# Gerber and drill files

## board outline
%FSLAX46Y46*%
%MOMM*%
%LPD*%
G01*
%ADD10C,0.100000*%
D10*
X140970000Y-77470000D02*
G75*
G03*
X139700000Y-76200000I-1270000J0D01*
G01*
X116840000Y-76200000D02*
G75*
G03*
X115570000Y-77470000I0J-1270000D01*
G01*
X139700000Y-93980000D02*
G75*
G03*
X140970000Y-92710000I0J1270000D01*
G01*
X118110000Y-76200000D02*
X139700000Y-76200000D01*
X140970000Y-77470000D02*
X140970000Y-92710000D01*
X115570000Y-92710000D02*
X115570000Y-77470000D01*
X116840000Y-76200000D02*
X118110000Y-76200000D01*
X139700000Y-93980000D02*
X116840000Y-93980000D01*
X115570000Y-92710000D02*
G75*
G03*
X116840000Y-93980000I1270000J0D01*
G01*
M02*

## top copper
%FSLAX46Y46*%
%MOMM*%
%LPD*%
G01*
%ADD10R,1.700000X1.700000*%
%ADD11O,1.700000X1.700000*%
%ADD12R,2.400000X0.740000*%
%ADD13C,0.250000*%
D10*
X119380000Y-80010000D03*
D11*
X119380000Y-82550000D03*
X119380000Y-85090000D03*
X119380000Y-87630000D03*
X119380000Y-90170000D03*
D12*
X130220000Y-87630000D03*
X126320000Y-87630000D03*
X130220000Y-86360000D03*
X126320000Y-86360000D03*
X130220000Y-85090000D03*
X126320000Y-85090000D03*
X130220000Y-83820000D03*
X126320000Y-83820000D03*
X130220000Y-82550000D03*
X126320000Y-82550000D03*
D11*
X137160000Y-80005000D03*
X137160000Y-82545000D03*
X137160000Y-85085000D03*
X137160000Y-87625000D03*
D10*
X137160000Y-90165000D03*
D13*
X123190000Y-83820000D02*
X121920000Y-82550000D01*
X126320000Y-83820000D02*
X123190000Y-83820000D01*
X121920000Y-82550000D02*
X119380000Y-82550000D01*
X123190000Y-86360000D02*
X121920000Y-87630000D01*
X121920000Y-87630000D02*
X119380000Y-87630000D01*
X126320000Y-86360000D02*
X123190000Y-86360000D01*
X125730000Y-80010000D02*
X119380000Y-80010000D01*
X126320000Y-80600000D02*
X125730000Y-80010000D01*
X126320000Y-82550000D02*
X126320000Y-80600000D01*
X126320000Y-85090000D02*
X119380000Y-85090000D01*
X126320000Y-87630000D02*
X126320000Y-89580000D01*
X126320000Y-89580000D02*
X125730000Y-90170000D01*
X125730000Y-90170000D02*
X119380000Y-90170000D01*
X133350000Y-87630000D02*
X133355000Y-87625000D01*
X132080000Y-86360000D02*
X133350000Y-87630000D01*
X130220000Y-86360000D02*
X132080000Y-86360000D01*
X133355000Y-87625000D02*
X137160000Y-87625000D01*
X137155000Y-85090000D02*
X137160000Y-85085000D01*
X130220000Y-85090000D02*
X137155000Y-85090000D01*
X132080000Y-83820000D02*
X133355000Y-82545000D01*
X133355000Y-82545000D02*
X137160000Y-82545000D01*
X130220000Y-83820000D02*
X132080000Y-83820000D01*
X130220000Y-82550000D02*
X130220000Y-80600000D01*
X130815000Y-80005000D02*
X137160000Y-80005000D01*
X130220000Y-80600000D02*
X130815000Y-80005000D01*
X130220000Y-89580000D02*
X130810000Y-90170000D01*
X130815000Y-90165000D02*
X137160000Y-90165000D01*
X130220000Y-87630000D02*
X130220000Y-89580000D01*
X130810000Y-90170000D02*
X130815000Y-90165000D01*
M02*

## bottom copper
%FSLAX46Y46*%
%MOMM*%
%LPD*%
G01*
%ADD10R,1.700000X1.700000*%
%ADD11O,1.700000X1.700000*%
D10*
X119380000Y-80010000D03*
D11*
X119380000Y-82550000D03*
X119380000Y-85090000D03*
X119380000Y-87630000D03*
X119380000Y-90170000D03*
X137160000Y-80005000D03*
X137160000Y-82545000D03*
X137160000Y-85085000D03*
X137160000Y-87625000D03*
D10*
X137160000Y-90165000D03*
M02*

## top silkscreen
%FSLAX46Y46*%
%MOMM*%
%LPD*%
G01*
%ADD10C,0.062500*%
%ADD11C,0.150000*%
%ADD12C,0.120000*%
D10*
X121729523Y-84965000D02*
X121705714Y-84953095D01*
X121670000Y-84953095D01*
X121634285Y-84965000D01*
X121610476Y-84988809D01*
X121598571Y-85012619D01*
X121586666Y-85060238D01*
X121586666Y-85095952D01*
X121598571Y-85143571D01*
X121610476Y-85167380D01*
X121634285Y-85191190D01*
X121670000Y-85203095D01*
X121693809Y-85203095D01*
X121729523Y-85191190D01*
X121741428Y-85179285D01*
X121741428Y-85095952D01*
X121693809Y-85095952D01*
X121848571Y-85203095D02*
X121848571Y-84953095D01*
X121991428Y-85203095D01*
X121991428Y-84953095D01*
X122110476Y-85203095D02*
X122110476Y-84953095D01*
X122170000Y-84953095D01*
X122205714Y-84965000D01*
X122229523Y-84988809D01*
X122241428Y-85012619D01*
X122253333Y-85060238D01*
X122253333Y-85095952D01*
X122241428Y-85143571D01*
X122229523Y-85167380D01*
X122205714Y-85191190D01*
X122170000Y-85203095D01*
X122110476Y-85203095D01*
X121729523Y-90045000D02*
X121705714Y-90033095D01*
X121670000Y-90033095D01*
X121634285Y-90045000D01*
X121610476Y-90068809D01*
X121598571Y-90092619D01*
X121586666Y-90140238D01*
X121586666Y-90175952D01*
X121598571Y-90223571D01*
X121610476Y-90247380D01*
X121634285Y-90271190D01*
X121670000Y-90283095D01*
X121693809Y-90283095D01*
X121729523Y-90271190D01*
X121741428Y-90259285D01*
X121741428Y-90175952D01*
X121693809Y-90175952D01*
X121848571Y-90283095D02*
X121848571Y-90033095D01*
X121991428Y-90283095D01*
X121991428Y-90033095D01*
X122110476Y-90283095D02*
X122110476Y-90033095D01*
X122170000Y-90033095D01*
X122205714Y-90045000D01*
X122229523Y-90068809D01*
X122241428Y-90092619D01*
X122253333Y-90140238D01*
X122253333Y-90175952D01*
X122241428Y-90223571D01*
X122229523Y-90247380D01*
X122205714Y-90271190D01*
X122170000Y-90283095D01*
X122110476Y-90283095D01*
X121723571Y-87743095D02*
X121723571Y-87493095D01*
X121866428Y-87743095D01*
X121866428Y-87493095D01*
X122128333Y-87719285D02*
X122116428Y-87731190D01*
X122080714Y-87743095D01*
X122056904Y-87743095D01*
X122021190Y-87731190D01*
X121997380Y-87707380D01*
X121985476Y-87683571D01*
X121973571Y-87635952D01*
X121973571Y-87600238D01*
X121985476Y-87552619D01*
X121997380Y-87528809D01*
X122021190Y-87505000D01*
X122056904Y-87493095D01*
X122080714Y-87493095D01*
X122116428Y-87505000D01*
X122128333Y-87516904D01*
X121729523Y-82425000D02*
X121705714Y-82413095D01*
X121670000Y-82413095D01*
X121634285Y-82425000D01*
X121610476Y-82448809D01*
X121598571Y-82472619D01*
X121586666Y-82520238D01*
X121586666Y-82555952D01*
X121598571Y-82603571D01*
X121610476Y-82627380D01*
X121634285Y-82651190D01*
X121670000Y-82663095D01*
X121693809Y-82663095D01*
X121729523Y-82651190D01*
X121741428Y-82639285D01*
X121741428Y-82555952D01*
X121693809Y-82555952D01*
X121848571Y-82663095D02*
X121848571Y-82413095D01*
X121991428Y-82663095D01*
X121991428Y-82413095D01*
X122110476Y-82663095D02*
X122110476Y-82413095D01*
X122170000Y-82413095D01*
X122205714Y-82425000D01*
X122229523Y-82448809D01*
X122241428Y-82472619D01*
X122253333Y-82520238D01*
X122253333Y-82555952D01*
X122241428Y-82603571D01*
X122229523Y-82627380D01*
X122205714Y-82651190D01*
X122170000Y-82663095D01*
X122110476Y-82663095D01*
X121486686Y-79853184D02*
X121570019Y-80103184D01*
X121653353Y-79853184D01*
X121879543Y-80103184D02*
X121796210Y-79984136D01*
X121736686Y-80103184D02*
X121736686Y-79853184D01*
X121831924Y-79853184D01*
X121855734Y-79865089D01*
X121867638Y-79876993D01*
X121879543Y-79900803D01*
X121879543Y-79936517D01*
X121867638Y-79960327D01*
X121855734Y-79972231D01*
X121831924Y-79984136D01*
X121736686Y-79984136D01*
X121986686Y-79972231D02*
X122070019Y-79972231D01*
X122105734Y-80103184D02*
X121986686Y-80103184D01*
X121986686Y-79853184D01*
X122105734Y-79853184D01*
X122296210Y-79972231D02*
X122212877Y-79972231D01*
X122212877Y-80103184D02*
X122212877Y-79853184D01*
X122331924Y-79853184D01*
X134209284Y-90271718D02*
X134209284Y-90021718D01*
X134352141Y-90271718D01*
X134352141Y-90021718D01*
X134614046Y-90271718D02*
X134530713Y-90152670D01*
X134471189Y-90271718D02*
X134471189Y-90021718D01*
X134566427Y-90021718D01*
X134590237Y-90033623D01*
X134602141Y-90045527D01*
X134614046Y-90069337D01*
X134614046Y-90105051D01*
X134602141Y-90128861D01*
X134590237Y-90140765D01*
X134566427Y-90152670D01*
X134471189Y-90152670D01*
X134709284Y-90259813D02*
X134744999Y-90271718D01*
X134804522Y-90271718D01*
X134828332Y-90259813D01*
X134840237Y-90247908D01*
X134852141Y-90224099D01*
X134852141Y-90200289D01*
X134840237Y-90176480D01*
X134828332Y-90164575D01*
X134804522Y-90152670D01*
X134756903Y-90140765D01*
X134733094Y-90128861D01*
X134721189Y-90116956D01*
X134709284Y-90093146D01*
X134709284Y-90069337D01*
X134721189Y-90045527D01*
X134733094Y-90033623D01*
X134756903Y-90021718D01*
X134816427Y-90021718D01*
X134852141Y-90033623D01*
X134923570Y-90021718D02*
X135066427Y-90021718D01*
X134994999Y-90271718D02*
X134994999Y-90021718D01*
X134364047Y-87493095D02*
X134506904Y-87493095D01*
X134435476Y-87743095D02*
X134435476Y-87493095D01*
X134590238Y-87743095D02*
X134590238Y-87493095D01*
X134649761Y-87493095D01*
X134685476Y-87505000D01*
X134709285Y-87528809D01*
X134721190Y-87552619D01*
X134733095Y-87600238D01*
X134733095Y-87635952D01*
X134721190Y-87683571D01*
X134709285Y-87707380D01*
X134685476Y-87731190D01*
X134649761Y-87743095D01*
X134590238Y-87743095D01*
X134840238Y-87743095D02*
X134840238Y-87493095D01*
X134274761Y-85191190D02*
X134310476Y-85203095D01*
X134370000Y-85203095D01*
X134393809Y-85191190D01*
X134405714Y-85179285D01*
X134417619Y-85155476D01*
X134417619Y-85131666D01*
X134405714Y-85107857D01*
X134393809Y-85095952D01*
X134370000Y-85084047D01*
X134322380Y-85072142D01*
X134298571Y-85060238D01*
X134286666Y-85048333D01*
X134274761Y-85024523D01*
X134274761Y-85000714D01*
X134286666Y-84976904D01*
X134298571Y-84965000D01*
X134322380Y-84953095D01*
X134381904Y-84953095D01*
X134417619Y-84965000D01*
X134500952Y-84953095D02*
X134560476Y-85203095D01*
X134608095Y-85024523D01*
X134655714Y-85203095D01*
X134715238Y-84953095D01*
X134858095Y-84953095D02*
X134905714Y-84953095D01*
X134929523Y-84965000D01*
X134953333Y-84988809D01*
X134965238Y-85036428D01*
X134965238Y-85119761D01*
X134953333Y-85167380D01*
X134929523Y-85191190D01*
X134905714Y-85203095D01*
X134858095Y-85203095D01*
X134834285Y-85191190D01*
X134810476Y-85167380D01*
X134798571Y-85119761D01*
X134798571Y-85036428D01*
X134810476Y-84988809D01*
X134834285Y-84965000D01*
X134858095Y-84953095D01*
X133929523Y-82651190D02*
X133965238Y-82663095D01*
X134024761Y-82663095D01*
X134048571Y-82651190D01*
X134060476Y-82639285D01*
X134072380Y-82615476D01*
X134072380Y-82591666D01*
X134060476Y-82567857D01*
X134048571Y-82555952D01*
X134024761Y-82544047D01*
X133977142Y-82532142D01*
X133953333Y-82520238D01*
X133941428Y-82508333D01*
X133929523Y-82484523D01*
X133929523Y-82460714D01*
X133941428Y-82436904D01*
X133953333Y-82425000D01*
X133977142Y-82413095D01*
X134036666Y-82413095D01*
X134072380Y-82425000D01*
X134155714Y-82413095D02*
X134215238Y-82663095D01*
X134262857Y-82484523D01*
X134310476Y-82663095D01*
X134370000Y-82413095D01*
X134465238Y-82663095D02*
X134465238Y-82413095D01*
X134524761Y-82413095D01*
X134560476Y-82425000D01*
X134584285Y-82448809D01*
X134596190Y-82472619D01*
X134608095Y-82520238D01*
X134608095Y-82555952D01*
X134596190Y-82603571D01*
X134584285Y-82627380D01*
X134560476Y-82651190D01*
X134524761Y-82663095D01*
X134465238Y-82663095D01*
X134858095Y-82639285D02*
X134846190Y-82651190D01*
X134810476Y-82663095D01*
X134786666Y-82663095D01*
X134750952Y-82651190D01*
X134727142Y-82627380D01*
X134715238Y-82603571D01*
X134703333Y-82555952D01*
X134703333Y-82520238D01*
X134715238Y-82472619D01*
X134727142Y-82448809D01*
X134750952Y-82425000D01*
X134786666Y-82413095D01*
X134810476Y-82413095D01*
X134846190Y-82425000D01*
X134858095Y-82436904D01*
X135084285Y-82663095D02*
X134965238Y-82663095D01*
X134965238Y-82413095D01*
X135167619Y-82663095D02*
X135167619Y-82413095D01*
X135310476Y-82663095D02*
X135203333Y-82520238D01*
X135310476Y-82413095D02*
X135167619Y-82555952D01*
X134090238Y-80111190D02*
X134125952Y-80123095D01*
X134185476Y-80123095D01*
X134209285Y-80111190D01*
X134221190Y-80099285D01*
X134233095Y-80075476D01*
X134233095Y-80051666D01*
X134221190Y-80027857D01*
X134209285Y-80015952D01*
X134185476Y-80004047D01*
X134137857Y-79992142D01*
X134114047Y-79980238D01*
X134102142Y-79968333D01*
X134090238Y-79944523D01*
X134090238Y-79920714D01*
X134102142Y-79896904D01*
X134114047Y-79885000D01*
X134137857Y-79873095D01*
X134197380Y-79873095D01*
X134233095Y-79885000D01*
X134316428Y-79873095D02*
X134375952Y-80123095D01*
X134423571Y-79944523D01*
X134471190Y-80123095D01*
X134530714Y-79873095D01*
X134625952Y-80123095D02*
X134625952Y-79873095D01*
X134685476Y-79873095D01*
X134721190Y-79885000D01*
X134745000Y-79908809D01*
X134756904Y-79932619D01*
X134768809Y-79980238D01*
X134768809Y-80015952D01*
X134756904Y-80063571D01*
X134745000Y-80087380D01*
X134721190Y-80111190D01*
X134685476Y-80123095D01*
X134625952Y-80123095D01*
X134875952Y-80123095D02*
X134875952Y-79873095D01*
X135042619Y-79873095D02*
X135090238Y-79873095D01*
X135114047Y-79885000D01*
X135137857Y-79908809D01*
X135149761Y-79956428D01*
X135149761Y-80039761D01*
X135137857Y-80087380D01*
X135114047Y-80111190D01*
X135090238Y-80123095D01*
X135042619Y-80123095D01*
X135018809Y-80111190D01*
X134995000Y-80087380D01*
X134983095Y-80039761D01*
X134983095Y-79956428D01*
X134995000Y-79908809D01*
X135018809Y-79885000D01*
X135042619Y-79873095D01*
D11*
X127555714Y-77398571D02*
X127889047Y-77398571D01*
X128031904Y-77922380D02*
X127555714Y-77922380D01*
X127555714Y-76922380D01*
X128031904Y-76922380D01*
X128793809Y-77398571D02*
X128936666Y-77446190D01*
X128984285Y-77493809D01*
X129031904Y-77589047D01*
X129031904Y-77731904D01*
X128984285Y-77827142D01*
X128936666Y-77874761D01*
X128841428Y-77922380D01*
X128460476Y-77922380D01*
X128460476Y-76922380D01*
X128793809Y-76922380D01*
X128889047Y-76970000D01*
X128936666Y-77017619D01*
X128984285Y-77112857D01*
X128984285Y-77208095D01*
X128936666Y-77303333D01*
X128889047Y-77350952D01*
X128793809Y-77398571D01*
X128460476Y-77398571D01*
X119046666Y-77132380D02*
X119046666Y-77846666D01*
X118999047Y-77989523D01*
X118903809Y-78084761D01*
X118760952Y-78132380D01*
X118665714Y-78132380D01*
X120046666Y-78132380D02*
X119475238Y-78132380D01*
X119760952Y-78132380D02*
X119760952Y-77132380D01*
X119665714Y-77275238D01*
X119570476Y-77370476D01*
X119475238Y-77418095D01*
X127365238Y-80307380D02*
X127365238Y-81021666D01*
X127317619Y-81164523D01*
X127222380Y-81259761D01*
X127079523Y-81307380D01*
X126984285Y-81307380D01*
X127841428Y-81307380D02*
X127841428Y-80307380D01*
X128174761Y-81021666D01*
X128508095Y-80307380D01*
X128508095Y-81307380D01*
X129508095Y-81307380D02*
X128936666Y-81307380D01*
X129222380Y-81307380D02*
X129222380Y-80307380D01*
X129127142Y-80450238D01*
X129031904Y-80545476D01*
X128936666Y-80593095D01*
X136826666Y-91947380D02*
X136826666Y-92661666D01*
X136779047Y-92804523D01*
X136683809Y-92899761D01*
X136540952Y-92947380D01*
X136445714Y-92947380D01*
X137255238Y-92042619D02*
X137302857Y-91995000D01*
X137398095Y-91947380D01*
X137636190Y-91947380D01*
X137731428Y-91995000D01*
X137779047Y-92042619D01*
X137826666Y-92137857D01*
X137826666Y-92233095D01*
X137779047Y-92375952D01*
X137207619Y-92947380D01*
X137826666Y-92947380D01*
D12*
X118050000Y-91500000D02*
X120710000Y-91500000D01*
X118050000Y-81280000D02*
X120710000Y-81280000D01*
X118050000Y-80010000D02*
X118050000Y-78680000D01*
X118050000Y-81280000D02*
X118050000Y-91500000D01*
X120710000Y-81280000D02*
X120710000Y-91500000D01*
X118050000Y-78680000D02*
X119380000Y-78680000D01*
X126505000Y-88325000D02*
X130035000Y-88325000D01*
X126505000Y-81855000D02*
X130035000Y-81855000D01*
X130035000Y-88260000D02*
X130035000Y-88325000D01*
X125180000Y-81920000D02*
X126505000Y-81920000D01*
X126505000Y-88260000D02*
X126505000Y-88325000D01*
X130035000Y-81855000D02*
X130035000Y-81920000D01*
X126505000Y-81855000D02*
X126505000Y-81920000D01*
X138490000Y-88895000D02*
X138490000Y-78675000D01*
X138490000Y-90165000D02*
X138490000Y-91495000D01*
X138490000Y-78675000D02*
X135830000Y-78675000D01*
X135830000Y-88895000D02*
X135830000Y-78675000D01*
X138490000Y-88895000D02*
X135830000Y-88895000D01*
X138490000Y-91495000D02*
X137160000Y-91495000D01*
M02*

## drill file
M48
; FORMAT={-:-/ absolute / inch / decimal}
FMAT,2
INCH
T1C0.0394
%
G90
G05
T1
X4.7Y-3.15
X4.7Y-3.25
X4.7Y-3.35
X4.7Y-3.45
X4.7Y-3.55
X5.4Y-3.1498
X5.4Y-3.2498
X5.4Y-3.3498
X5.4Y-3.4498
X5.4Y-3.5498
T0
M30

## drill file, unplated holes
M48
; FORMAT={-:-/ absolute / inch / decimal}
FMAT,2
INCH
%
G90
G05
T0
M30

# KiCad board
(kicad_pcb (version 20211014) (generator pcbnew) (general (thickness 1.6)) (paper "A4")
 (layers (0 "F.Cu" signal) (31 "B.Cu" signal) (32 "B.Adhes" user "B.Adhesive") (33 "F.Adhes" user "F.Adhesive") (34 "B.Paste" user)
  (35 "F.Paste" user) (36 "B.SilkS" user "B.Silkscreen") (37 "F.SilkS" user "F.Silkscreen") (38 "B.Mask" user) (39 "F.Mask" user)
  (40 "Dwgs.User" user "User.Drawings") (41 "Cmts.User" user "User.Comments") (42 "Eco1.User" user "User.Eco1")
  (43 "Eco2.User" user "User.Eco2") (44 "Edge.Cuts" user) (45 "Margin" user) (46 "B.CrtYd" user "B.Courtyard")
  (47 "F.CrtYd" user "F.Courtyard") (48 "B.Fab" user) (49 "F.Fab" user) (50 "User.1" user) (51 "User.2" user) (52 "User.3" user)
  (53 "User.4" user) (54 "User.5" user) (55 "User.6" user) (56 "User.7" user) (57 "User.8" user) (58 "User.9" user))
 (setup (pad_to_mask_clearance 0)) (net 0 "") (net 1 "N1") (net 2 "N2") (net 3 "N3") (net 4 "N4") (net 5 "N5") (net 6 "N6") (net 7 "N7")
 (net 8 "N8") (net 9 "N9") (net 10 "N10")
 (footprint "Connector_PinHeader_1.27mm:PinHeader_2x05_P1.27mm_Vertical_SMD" (layer "F.Cu") (at 128.27 85.09)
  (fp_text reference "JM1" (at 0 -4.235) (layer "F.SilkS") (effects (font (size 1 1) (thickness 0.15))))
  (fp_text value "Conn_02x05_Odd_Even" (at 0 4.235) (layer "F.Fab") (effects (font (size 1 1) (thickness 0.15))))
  (fp_line (start -1.765 -3.235) (end -1.765 -3.17) (layer "F.SilkS") (width 0.12))
  (fp_line (start 1.765 -3.235) (end 1.765 -3.17) (layer "F.SilkS") (width 0.12))
  (fp_line (start -1.765 3.17) (end -1.765 3.235) (layer "F.SilkS") (width 0.12))
  (fp_line (start -3.09 -3.17) (end -1.765 -3.17) (layer "F.SilkS") (width 0.12))
  (fp_line (start 1.765 3.17) (end 1.765 3.235) (layer "F.SilkS") (width 0.12))
  (fp_line (start -1.765 -3.235) (end 1.765 -3.235) (layer "F.SilkS") (width 0.12))
  (fp_line (start -1.765 3.235) (end 1.765 3.235) (layer "F.SilkS") (width 0.12))
  (pad "1" smd rect (at -1.95 -2.54) (size 2.4 0.74) (layers "F.Cu" "F.Paste" "F.Mask") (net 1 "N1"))
  (pad "2" smd rect (at 1.95 -2.54) (size 2.4 0.74) (layers "F.Cu" "F.Paste" "F.Mask") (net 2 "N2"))
  (pad "3" smd rect (at -1.95 -1.27) (size 2.4 0.74) (layers "F.Cu" "F.Paste" "F.Mask") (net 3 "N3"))
  (pad "4" smd rect (at 1.95 -1.27) (size 2.4 0.74) (layers "F.Cu" "F.Paste" "F.Mask") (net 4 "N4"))
  (pad "5" smd rect (at -1.95 0) (size 2.4 0.74) (layers "F.Cu" "F.Paste" "F.Mask") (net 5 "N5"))
  (pad "6" smd rect (at 1.95 0) (size 2.4 0.74) (layers "F.Cu" "F.Paste" "F.Mask") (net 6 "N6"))
  (pad "7" smd rect (at -1.95 1.27) (size 2.4 0.74) (layers "F.Cu" "F.Paste" "F.Mask") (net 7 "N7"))
  (pad "8" smd rect (at 1.95 1.27) (size 2.4 0.74) (layers "F.Cu" "F.Paste" "F.Mask") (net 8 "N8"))
  (pad "9" smd rect (at -1.95 2.54) (size 2.4 0.74) (layers "F.Cu" "F.Paste" "F.Mask") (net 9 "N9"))
  (pad "10" smd rect (at 1.95 2.54) (size 2.4 0.74) (layers "F.Cu" "F.Paste" "F.Mask") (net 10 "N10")))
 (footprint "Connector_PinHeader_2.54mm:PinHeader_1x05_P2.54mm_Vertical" (layer "F.Cu") (at 119.38 80.01)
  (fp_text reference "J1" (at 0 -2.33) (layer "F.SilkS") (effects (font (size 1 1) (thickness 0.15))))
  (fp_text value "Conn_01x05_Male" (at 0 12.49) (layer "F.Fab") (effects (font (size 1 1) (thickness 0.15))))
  (fp_line (start -1.33 11.49) (end 1.33 11.49) (layer "F.SilkS") (width 0.12))
  (fp_line (start -1.33 1.27) (end 1.33 1.27) (layer "F.SilkS") (width 0.12))
  (fp_line (start -1.33 0) (end -1.33 -1.33) (layer "F.SilkS") (width 0.12))
  (fp_line (start -1.33 1.27) (end -1.33 11.49) (layer "F.SilkS") (width 0.12))
  (fp_line (start 1.33 1.27) (end 1.33 11.49) (layer "F.SilkS") (width 0.12))
  (fp_line (start -1.33 -1.33) (end 0 -1.33) (layer "F.SilkS") (width 0.12))
  (pad "1" thru_hole rect (at 0 0) (size 1.7 1.7) (drill 1) (layers *.Cu *.Mask) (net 1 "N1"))
  (pad "2" thru_hole oval (at 0 2.54) (size 1.7 1.7) (drill 1) (layers *.Cu *.Mask) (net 3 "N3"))
  (pad "3" thru_hole oval (at 0 5.08) (size 1.7 1.7) (drill 1) (layers *.Cu *.Mask) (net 5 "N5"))
  (pad "4" thru_hole oval (at 0 7.62) (size 1.7 1.7) (drill 1) (layers *.Cu *.Mask) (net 7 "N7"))
  (pad "5" thru_hole oval (at 0 10.16) (size 1.7 1.7) (drill 1) (layers *.Cu *.Mask) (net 9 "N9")))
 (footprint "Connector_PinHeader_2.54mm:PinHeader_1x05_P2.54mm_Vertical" (layer "F.Cu") (at 137.16 90.165 180)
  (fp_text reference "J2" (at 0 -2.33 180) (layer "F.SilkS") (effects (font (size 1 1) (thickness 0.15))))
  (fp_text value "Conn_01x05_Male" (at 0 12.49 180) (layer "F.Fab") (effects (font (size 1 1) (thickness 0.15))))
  (fp_line (start -1.33 -1.33) (end 0 -1.33) (layer "F.SilkS") (width 0.12))
  (fp_line (start -1.33 1.27) (end 1.33 1.27) (layer "F.SilkS") (width 0.12))
  (fp_line (start 1.33 1.27) (end 1.33 11.49) (layer "F.SilkS") (width 0.12))
  (fp_line (start -1.33 11.49) (end 1.33 11.49) (layer "F.SilkS") (width 0.12))
  (fp_line (start -1.33 0) (end -1.33 -1.33) (layer "F.SilkS") (width 0.12))
  (fp_line (start -1.33 1.27) (end -1.33 11.49) (layer "F.SilkS") (width 0.12))
  (pad "1" thru_hole rect (at 0 0 180) (size 1.7 1.7) (drill 1) (layers *.Cu *.Mask) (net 10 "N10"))
  (pad "2" thru_hole oval (at 0 2.54 180) (size 1.7 1.7) (drill 1) (layers *.Cu *.Mask) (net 8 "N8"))
  (pad "3" thru_hole oval (at 0 5.08 180) (size 1.7 1.7) (drill 1) (layers *.Cu *.Mask) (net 6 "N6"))
  (pad "4" thru_hole oval (at 0 7.62 180) (size 1.7 1.7) (drill 1) (layers *.Cu *.Mask) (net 4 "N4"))
  (pad "5" thru_hole oval (at 0 10.16 180) (size 1.7 1.7) (drill 1) (layers *.Cu *.Mask) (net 2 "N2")))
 (gr_arc (start 139.7 76.2) (mid 140.598026 76.571974) (end 140.97 77.47) (layer "Edge.Cuts") (width 0.1))
 (gr_arc (start 115.57 77.47) (mid 115.941974 76.571974) (end 116.84 76.2) (layer "Edge.Cuts") (width 0.1))
 (gr_arc (start 140.97 92.71) (mid 140.598026 93.608026) (end 139.7 93.98) (layer "Edge.Cuts") (width 0.1))
 (gr_line (start 118.11 76.2) (end 139.7 76.2) (layer "Edge.Cuts") (width 0.1))
 (gr_line (start 140.97 77.47) (end 140.97 92.71) (layer "Edge.Cuts") (width 0.1))
 (gr_line (start 115.57 92.71) (end 115.57 77.47) (layer "Edge.Cuts") (width 0.1))
 (gr_line (start 116.84 76.2) (end 118.11 76.2) (layer "Edge.Cuts") (width 0.1))
 (gr_line (start 139.7 93.98) (end 116.84 93.98) (layer "Edge.Cuts") (width 0.1))
 (gr_arc (start 116.84 93.98) (mid 115.941974 93.608026) (end 115.57 92.71) (layer "Edge.Cuts") (width 0.1))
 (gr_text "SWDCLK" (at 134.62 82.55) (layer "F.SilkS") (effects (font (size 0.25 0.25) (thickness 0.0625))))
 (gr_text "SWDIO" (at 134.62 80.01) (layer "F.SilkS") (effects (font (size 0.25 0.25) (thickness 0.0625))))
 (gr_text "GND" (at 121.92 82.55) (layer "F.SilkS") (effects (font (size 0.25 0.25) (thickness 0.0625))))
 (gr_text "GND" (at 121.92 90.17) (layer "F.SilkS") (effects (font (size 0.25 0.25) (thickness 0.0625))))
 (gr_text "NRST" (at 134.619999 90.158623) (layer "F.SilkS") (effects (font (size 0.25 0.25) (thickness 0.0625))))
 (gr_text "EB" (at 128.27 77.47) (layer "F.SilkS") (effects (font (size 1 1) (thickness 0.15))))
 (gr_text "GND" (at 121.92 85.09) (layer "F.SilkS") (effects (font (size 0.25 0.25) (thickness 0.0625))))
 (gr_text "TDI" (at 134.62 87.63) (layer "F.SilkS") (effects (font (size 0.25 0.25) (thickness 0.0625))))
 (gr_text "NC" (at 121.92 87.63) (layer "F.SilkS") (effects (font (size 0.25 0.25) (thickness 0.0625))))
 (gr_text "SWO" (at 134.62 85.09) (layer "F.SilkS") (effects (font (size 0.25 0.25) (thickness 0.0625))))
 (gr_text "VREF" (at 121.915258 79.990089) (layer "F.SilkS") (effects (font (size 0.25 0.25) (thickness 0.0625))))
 (segment (start 123.19 83.82) (end 121.92 82.55) (width 0.25) (layer "F.Cu") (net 3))
 (segment (start 126.32 83.82) (end 123.19 83.82) (width 0.25) (layer "F.Cu") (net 3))
 (segment (start 121.92 82.55) (end 119.38 82.55) (width 0.25) (layer "F.Cu") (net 3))
 (segment (start 123.19 86.36) (end 121.92 87.63) (width 0.25) (layer "F.Cu") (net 7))
 (segment (start 121.92 87.63) (end 119.38 87.63) (width 0.25) (layer "F.Cu") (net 7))
 (segment (start 126.32 86.36) (end 123.19 86.36) (width 0.25) (layer "F.Cu") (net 7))
 (segment (start 125.73 80.01) (end 119.38 80.01) (width 0.25) (layer "F.Cu") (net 1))
 (segment (start 126.32 80.6) (end 125.73 80.01) (width 0.25) (layer "F.Cu") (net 1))
 (segment (start 126.32 82.55) (end 126.32 80.6) (width 0.25) (layer "F.Cu") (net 1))
 (segment (start 126.32 85.09) (end 119.38 85.09) (width 0.25) (layer "F.Cu") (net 5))
 (segment (start 126.32 87.63) (end 126.32 89.58) (width 0.25) (layer "F.Cu") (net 9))
 (segment (start 126.32 89.58) (end 125.73 90.17) (width 0.25) (layer "F.Cu") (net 9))
 (segment (start 125.73 90.17) (end 119.38 90.17) (width 0.25) (layer "F.Cu") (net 9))
 (segment (start 130.22 82.55) (end 130.22 80.6) (width 0.25) (layer "F.Cu") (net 2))
 (segment (start 130.815 80.005) (end 137.16 80.005) (width 0.25) (layer "F.Cu") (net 2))
 (segment (start 130.22 80.6) (end 130.815 80.005) (width 0.25) (layer "F.Cu") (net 2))
 (segment (start 132.08 83.82) (end 133.355 82.545) (width 0.25) (layer "F.Cu") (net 4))
 (segment (start 133.355 82.545) (end 137.16 82.545) (width 0.25) (layer "F.Cu") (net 4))
 (segment (start 130.22 83.82) (end 132.08 83.82) (width 0.25) (layer "F.Cu") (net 4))
 (segment (start 137.155 85.09) (end 137.16 85.085) (width 0.25) (layer "F.Cu") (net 6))
 (segment (start 130.22 85.09) (end 137.155 85.09) (width 0.25) (layer "F.Cu") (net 6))
 (segment (start 133.35 87.63) (end 133.355 87.625) (width 0.25) (layer "F.Cu") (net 8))
 (segment (start 132.08 86.36) (end 133.35 87.63) (width 0.25) (layer "F.Cu") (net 8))
 (segment (start 130.22 86.36) (end 132.08 86.36) (width 0.25) (layer "F.Cu") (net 8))
 (segment (start 133.355 87.625) (end 137.16 87.625) (width 0.25) (layer "F.Cu") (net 8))
 (segment (start 130.22 89.58) (end 130.81 90.17) (width 0.25) (layer "F.Cu") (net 10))
 (segment (start 130.815 90.165) (end 137.16 90.165) (width 0.25) (layer "F.Cu") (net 10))
 (segment (start 130.22 87.63) (end 130.22 89.58) (width 0.25) (layer "F.Cu") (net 10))
 (segment (start 130.81 90.17) (end 130.815 90.165) (width 0.25) (layer "F.Cu") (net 10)))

